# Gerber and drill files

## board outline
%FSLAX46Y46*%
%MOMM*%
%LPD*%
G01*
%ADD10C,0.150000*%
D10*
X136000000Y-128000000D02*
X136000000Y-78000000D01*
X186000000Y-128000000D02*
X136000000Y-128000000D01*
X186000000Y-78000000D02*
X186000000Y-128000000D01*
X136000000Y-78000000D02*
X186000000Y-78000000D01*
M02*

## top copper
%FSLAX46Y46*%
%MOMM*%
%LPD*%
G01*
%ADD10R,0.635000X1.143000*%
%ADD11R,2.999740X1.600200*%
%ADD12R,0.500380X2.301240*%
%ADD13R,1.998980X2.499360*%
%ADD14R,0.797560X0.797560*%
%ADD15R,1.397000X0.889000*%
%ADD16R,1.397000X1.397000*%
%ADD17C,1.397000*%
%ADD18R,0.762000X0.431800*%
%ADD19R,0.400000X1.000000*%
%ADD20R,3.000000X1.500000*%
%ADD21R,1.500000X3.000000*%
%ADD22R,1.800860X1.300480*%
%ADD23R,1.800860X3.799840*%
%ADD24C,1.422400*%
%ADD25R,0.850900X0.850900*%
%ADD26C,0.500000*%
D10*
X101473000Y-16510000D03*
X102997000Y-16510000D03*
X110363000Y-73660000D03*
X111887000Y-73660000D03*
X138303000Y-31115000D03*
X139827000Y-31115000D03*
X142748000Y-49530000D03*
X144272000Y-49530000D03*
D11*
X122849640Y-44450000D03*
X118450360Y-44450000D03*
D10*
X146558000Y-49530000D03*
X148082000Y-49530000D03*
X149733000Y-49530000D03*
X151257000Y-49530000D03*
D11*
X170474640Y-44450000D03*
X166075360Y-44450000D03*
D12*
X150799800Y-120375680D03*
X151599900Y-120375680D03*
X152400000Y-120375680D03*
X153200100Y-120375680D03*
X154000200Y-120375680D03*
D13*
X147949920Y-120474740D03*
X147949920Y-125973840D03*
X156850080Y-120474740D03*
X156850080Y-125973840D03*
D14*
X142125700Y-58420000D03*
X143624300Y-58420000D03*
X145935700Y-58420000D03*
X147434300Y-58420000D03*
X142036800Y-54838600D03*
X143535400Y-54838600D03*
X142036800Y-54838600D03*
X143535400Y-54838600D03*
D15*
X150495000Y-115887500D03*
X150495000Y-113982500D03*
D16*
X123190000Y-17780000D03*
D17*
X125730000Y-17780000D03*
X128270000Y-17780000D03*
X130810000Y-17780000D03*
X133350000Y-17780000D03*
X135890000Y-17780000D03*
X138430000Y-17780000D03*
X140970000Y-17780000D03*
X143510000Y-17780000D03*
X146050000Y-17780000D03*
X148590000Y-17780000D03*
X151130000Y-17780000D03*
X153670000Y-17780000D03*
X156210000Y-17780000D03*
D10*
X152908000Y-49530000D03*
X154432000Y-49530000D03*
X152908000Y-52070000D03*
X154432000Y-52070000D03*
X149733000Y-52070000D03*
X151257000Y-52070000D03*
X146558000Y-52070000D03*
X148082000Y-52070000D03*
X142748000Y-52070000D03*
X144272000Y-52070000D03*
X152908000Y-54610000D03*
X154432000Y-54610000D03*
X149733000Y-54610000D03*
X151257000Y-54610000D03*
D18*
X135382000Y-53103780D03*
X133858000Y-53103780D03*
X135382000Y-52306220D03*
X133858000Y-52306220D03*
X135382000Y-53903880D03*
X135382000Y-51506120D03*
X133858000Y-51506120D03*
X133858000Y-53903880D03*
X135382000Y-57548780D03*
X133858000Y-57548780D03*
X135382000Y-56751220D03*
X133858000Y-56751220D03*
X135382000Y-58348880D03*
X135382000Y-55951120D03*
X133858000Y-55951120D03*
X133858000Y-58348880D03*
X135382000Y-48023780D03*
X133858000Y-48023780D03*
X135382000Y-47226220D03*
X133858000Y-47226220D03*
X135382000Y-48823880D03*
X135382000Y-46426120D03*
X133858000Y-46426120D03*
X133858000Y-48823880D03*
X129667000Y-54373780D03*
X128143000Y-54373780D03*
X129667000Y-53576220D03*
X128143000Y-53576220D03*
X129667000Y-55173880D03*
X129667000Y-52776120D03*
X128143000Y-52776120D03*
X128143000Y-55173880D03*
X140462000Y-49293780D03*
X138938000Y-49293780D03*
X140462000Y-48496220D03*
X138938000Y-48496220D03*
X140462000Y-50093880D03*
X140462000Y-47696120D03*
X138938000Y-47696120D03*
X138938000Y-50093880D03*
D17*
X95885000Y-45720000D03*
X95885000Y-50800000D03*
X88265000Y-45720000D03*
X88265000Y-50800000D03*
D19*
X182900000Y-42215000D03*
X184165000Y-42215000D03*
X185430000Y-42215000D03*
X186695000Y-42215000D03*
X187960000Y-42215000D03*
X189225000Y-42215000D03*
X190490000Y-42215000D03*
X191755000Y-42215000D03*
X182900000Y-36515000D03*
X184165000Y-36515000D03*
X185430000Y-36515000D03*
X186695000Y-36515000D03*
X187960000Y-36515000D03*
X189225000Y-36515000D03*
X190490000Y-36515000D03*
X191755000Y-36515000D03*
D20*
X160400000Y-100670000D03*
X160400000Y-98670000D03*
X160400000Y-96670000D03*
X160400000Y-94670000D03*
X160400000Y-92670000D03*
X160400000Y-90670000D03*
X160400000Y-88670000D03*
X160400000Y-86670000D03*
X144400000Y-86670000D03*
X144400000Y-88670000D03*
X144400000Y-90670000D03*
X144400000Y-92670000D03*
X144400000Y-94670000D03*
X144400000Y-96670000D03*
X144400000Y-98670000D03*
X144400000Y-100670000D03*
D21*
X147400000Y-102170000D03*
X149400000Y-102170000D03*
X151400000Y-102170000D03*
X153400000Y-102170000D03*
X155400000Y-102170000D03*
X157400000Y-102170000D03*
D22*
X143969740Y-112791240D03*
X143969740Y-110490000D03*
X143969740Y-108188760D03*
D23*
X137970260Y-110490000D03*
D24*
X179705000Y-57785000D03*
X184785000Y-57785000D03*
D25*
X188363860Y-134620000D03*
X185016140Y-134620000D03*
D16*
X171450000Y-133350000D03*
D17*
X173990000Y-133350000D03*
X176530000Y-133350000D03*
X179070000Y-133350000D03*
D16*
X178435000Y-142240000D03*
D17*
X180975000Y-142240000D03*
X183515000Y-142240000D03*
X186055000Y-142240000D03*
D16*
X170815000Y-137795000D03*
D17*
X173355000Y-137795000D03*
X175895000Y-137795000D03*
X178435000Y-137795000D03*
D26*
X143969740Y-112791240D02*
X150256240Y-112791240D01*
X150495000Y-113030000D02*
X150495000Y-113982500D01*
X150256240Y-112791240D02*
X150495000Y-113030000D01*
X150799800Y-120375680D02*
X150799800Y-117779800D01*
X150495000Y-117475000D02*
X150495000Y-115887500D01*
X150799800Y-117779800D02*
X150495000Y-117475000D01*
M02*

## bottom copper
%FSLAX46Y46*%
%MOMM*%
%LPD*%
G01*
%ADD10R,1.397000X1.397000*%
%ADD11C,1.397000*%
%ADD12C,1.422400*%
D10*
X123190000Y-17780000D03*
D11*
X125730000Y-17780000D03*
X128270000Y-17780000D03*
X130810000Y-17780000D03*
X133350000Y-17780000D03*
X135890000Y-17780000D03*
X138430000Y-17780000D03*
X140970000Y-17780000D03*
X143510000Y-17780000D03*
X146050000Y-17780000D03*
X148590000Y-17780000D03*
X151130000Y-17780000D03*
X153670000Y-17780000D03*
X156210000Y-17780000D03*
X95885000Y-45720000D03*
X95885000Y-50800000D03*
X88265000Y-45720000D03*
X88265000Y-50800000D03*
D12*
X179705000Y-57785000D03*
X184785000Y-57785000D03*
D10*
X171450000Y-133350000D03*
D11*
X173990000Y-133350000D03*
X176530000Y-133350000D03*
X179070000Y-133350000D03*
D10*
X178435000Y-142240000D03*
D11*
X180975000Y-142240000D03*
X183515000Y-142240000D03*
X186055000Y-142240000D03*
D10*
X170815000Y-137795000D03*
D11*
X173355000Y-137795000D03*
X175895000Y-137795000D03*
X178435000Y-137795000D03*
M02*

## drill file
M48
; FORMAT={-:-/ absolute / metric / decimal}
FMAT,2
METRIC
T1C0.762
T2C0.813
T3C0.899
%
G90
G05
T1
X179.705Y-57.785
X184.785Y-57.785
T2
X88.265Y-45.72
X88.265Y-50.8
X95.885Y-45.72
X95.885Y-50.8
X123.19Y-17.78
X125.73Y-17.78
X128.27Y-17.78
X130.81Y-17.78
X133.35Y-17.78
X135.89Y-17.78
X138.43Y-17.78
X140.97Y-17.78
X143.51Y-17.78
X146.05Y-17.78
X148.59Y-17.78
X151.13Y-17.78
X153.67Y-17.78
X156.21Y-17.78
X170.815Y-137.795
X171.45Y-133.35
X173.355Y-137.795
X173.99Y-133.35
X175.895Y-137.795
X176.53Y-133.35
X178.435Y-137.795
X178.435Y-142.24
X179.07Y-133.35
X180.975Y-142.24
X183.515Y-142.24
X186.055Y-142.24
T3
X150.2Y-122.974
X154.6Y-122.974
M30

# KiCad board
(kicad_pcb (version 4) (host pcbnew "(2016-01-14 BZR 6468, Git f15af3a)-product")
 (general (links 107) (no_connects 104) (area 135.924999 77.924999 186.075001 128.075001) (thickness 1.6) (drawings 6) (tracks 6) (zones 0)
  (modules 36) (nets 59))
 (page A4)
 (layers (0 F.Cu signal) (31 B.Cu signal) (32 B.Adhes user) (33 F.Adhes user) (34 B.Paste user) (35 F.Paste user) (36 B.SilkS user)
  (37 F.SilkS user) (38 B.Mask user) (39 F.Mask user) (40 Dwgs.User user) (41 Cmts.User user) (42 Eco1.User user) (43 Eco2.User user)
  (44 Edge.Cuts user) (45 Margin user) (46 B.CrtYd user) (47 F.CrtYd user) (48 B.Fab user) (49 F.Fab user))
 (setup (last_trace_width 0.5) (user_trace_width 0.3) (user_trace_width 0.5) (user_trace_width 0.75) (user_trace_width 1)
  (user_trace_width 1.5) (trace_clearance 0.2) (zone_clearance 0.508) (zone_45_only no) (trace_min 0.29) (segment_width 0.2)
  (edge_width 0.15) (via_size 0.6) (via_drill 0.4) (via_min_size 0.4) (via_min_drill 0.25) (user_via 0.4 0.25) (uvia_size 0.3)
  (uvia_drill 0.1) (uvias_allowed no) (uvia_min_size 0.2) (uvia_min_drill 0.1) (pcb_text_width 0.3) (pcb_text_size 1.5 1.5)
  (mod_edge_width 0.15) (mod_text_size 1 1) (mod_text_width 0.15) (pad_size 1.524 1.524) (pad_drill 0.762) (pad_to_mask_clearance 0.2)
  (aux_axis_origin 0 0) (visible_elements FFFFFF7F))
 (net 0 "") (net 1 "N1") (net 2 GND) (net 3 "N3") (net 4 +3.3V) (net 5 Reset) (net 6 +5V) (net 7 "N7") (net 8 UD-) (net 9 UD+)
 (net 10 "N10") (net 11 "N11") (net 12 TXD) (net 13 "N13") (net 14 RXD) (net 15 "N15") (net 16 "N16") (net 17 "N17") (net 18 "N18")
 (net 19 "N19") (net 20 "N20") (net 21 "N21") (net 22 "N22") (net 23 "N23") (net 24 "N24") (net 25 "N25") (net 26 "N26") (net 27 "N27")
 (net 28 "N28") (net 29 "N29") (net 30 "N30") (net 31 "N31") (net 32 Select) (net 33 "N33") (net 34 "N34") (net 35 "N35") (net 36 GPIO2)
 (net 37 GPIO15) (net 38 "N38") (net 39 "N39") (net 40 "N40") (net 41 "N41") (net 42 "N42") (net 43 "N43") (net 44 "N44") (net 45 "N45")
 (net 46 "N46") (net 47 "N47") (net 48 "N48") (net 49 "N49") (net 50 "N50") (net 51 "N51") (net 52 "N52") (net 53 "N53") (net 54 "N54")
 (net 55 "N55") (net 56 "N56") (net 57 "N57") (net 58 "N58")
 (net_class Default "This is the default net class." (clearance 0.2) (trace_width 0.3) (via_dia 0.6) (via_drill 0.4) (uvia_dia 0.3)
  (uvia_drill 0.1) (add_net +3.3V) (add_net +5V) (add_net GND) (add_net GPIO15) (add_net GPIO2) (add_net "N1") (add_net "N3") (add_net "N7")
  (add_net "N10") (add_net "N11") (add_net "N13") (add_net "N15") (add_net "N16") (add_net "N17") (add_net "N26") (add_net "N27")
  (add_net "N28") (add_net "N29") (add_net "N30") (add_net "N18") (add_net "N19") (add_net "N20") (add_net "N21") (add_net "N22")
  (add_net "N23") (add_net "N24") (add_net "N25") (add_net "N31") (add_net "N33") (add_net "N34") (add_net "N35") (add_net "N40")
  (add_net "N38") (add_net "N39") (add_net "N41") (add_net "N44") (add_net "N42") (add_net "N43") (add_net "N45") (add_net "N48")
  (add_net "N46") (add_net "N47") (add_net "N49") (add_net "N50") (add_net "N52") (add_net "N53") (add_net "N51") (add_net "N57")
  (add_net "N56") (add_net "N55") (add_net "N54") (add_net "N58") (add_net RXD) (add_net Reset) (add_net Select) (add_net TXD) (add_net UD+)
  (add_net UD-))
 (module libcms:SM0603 (layer F.Cu) (at 102.235 16.51)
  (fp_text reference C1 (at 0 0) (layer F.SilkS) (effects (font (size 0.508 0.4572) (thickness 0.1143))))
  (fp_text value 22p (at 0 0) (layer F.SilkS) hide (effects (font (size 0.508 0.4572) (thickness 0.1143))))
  (pad 1 smd rect (at -0.762 0) (size 0.635 1.143) (layers F.Cu F.Paste F.Mask) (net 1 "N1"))
  (pad 2 smd rect (at 0.762 0) (size 0.635 1.143) (layers F.Cu F.Paste F.Mask) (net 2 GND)))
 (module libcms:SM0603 (layer F.Cu) (at 111.125 73.66)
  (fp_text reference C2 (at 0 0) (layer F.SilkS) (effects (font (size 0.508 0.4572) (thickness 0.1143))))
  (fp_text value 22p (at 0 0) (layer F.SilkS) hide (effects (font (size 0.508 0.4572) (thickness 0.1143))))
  (pad 1 smd rect (at -0.762 0) (size 0.635 1.143) (layers F.Cu F.Paste F.Mask) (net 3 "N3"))
  (pad 2 smd rect (at 0.762 0) (size 0.635 1.143) (layers F.Cu F.Paste F.Mask) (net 2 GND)))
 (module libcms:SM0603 (layer F.Cu) (at 139.065 31.115)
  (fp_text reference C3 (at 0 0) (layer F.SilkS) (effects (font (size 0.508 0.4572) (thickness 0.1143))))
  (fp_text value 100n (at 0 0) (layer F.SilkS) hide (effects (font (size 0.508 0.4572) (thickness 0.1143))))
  (pad 1 smd rect (at -0.762 0) (size 0.635 1.143) (layers F.Cu F.Paste F.Mask) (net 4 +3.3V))
  (pad 2 smd rect (at 0.762 0) (size 0.635 1.143) (layers F.Cu F.Paste F.Mask) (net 2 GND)))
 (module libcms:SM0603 (layer F.Cu) (at 143.51 49.53)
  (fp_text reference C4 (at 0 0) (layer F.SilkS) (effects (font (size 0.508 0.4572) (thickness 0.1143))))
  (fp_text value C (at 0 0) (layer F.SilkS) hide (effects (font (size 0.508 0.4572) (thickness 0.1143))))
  (pad 1 smd rect (at -0.762 0) (size 0.635 1.143) (layers F.Cu F.Paste F.Mask) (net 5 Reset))
  (pad 2 smd rect (at 0.762 0) (size 0.635 1.143) (layers F.Cu F.Paste F.Mask) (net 2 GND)))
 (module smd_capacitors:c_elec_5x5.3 (layer F.Cu) (at 120.65 44.45)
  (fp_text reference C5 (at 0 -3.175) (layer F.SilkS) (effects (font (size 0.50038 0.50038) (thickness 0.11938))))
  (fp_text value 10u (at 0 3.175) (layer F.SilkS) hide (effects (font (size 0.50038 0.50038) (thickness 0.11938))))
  (pad 1 smd rect (at 2.19964 0) (size 2.99974 1.6002) (layers F.Cu F.Paste F.Mask) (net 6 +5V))
  (pad 2 smd rect (at -2.19964 0) (size 2.99974 1.6002) (layers F.Cu F.Paste F.Mask) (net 2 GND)))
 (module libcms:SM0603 (layer F.Cu) (at 147.32 49.53)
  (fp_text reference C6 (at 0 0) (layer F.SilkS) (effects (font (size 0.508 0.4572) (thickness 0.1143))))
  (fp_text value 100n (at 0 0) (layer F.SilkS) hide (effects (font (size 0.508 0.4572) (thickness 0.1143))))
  (pad 1 smd rect (at -0.762 0) (size 0.635 1.143) (layers F.Cu F.Paste F.Mask) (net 6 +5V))
  (pad 2 smd rect (at 0.762 0) (size 0.635 1.143) (layers F.Cu F.Paste F.Mask) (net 2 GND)))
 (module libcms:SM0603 (layer F.Cu) (at 150.495 49.53)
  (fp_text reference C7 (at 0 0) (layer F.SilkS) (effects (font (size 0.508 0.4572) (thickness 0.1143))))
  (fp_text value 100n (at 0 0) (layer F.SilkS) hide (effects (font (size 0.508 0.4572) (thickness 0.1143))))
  (pad 1 smd rect (at -0.762 0) (size 0.635 1.143) (layers F.Cu F.Paste F.Mask) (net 4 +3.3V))
  (pad 2 smd rect (at 0.762 0) (size 0.635 1.143) (layers F.Cu F.Paste F.Mask) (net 2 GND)))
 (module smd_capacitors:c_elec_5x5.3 (layer F.Cu) (at 168.275 44.45)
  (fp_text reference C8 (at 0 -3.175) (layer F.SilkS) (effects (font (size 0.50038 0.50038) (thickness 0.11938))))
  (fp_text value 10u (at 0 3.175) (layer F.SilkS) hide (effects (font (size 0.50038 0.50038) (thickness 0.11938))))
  (pad 1 smd rect (at 2.19964 0) (size 2.99974 1.6002) (layers F.Cu F.Paste F.Mask) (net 4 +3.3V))
  (pad 2 smd rect (at -2.19964 0) (size 2.99974 1.6002) (layers F.Cu F.Paste F.Mask) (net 2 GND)))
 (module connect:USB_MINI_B (layer F.Cu) (at 152.4 123.825 90)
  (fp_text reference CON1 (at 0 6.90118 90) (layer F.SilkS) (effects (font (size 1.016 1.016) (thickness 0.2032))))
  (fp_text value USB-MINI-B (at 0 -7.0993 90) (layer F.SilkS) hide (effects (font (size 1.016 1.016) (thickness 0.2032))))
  (pad 1 smd rect (at 3.44932 -1.6002 90) (size 2.30124 0.50038) (layers F.Cu F.Paste F.Mask) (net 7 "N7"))
  (pad 2 smd rect (at 3.44932 -0.8001 90) (size 2.30124 0.50038) (layers F.Cu F.Paste F.Mask) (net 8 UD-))
  (pad 3 smd rect (at 3.44932 0 90) (size 2.30124 0.50038) (layers F.Cu F.Paste F.Mask) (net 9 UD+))
  (pad 4 smd rect (at 3.44932 0.8001 90) (size 2.30124 0.50038) (layers F.Cu F.Paste F.Mask) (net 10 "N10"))
  (pad 5 smd rect (at 3.44932 1.6002 90) (size 2.30124 0.50038) (layers F.Cu F.Paste F.Mask) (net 2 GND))
  (pad 6 smd rect (at 3.35026 -4.45008 90) (size 2.49936 1.99898) (layers F.Cu F.Paste F.Mask) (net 2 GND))
  (pad 7 smd rect (at -2.14884 -4.45008 90) (size 2.49936 1.99898) (layers F.Cu F.Paste F.Mask) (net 2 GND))
  (pad 8 smd rect (at 3.35026 4.45008 90) (size 2.49936 1.99898) (layers F.Cu F.Paste F.Mask) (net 2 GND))
  (pad 9 smd rect (at -2.14884 4.45008 90) (size 2.49936 1.99898) (layers F.Cu F.Paste F.Mask) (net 2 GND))
  (pad "" np_thru_hole circle (at 0.8509 -2.19964 90) (size 0.89916 0.89916) (drill 0.89916) (layers *.Cu *.Mask F.SilkS))
  (pad 2 np_thru_hole circle (at 0.8509 2.19964 90) (size 0.89916 0.89916) (drill 0.89916) (layers *.Cu *.Mask F.SilkS) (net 8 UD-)))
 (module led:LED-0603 (layer F.Cu) (at 142.875 58.42)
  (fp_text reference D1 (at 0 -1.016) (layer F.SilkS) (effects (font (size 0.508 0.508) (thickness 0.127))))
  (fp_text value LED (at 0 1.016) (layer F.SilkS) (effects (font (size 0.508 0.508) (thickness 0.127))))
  (pad 1 smd rect (at -0.7493 0) (size 0.79756 0.79756) (layers F.Cu F.Paste F.Mask) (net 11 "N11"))
  (pad 2 smd rect (at 0.7493 0) (size 0.79756 0.79756) (layers F.Cu F.Paste F.Mask) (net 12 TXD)))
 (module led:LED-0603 (layer F.Cu) (at 146.685 58.42)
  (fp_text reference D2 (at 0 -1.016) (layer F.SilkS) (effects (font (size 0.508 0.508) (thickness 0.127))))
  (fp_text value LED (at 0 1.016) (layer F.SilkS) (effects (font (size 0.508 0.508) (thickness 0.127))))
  (pad 1 smd rect (at -0.7493 0) (size 0.79756 0.79756) (layers F.Cu F.Paste F.Mask) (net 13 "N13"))
  (pad 2 smd rect (at 0.7493 0) (size 0.79756 0.79756) (layers F.Cu F.Paste F.Mask) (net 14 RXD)))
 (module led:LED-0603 (layer F.Cu) (at 142.7861 54.8386)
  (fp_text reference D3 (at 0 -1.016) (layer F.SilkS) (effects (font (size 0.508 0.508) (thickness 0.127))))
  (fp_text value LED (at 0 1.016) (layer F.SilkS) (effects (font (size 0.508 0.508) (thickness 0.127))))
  (pad 1 smd rect (at -0.7493 0) (size 0.79756 0.79756) (layers F.Cu F.Paste F.Mask) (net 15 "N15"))
  (pad 2 smd rect (at 0.7493 0) (size 0.79756 0.79756) (layers F.Cu F.Paste F.Mask) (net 2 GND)))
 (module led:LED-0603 (layer F.Cu) (at 142.7861 54.8386)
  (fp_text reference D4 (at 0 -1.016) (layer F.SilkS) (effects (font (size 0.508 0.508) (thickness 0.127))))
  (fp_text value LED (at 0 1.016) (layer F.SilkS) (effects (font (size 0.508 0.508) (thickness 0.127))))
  (pad 1 smd rect (at -0.7493 0) (size 0.79756 0.79756) (layers F.Cu F.Paste F.Mask) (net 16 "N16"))
  (pad 2 smd rect (at 0.7493 0) (size 0.79756 0.79756) (layers F.Cu F.Paste F.Mask) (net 2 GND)))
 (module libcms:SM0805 (layer F.Cu) (at 150.495 114.935 90)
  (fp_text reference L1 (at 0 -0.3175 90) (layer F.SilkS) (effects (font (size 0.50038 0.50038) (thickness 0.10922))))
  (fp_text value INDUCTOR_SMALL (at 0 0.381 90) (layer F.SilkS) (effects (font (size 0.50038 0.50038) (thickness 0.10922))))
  (pad 1 smd rect (at -0.9525 0 90) (size 0.889 1.397) (layers F.Cu F.Paste F.Mask) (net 7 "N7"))
  (pad 2 smd rect (at 0.9525 0 90) (size 0.889 1.397) (layers F.Cu F.Paste F.Mask) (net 6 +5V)))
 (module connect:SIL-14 (layer F.Cu) (at 139.7 17.78)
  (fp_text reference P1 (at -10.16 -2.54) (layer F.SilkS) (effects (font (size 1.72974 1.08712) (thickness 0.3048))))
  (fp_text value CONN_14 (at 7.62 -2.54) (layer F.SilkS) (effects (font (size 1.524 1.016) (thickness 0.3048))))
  (pad 1 thru_hole rect (at -16.51 0) (size 1.397 1.397) (drill 0.8128) (layers *.Cu *.Mask F.SilkS) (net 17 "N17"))
  (pad 2 thru_hole circle (at -13.97 0) (size 1.397 1.397) (drill 0.8128) (layers *.Cu *.Mask F.SilkS) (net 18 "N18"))
  (pad 3 thru_hole circle (at -11.43 0) (size 1.397 1.397) (drill 0.8128) (layers *.Cu *.Mask F.SilkS) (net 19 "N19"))
  (pad 4 thru_hole circle (at -8.89 0) (size 1.397 1.397) (drill 0.8128) (layers *.Cu *.Mask F.SilkS) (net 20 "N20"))
  (pad 5 thru_hole circle (at -6.35 0) (size 1.397 1.397) (drill 0.8128) (layers *.Cu *.Mask F.SilkS) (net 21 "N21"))
  (pad 6 thru_hole circle (at -3.81 0) (size 1.397 1.397) (drill 0.8128) (layers *.Cu *.Mask F.SilkS) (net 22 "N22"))
  (pad 7 thru_hole circle (at -1.27 0) (size 1.397 1.397) (drill 0.8128) (layers *.Cu *.Mask F.SilkS) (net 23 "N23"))
  (pad 8 thru_hole circle (at 1.27 0) (size 1.397 1.397) (drill 0.8128) (layers *.Cu *.Mask F.SilkS) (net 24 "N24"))
  (pad 9 thru_hole circle (at 3.81 0) (size 1.397 1.397) (drill 0.8128) (layers *.Cu *.Mask F.SilkS) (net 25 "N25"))
  (pad 10 thru_hole circle (at 6.35 0) (size 1.397 1.397) (drill 0.8128) (layers *.Cu *.Mask F.SilkS) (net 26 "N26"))
  (pad 11 thru_hole circle (at 8.89 0) (size 1.397 1.397) (drill 0.8128) (layers *.Cu *.Mask F.SilkS) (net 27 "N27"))
  (pad 12 thru_hole circle (at 11.43 0) (size 1.397 1.397) (drill 0.8128) (layers *.Cu *.Mask F.SilkS) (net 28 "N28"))
  (pad 13 thru_hole circle (at 13.97 0) (size 1.397 1.397) (drill 0.8128) (layers *.Cu *.Mask F.SilkS) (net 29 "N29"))
  (pad 14 thru_hole circle (at 16.51 0) (size 1.397 1.397) (drill 0.8128) (layers *.Cu *.Mask F.SilkS) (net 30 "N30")))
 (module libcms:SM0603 (layer F.Cu) (at 153.67 49.53)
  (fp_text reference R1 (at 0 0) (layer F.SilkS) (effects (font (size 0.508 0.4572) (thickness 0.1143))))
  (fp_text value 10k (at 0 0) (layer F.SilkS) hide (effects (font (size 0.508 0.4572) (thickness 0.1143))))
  (pad 1 smd rect (at -0.762 0) (size 0.635 1.143) (layers F.Cu F.Paste F.Mask) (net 5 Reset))
  (pad 2 smd rect (at 0.762 0) (size 0.635 1.143) (layers F.Cu F.Paste F.Mask) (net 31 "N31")))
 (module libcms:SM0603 (layer F.Cu) (at 153.67 52.07)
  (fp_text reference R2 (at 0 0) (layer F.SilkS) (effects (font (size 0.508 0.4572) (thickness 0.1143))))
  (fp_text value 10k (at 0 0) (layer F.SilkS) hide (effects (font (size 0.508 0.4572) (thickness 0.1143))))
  (pad 1 smd rect (at -0.762 0) (size 0.635 1.143) (layers F.Cu F.Paste F.Mask) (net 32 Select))
  (pad 2 smd rect (at 0.762 0) (size 0.635 1.143) (layers F.Cu F.Paste F.Mask) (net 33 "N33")))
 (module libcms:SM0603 (layer F.Cu) (at 150.495 52.07)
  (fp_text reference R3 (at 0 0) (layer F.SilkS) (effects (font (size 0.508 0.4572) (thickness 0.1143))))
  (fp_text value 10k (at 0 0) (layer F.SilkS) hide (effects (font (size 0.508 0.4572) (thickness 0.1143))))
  (pad 1 smd rect (at -0.762 0) (size 0.635 1.143) (layers F.Cu F.Paste F.Mask) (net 5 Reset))
  (pad 2 smd rect (at 0.762 0) (size 0.635 1.143) (layers F.Cu F.Paste F.Mask) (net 4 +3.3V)))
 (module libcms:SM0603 (layer F.Cu) (at 147.32 52.07)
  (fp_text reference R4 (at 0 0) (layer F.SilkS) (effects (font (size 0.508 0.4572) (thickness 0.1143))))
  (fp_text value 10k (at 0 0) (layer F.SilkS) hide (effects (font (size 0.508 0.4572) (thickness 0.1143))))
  (pad 1 smd rect (at -0.762 0) (size 0.635 1.143) (layers F.Cu F.Paste F.Mask) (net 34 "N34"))
  (pad 2 smd rect (at 0.762 0) (size 0.635 1.143) (layers F.Cu F.Paste F.Mask) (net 5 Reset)))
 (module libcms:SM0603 (layer F.Cu) (at 143.51 52.07)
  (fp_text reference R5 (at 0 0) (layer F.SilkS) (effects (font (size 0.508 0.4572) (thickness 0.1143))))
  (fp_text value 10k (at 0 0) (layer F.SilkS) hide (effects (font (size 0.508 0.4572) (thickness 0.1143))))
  (pad 1 smd rect (at -0.762 0) (size 0.635 1.143) (layers F.Cu F.Paste F.Mask) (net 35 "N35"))
  (pad 2 smd rect (at 0.762 0) (size 0.635 1.143) (layers F.Cu F.Paste F.Mask) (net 4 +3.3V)))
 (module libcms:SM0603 (layer F.Cu) (at 153.67 54.61)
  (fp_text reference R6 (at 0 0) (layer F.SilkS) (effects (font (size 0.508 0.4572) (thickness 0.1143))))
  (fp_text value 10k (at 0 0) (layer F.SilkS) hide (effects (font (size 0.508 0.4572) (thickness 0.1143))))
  (pad 1 smd rect (at -0.762 0) (size 0.635 1.143) (layers F.Cu F.Paste F.Mask) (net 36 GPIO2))
  (pad 2 smd rect (at 0.762 0) (size 0.635 1.143) (layers F.Cu F.Paste F.Mask) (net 4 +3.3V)))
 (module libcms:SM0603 (layer F.Cu) (at 150.495 54.61)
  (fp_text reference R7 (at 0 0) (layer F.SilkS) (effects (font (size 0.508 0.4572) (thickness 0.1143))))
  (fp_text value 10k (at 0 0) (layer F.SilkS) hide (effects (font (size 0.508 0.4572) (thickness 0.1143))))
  (pad 1 smd rect (at -0.762 0) (size 0.635 1.143) (layers F.Cu F.Paste F.Mask) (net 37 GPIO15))
  (pad 2 smd rect (at 0.762 0) (size 0.635 1.143) (layers F.Cu F.Paste F.Mask) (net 2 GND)))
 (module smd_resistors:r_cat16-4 (layer F.Cu) (at 134.62 52.705)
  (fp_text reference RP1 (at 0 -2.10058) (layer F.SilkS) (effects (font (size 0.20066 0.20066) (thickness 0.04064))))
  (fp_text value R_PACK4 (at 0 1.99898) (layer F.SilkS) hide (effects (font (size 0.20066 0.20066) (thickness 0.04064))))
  (pad 2 smd rect (at 0.762 0.39878) (size 0.762 0.4318) (layers F.Cu F.Paste F.Mask) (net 4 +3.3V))
  (pad 7 smd rect (at -0.762 0.39878) (size 0.762 0.4318) (layers F.Cu F.Paste F.Mask) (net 15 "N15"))
  (pad 3 smd rect (at 0.762 -0.39878) (size 0.762 0.4318) (layers F.Cu F.Paste F.Mask) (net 4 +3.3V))
  (pad 6 smd rect (at -0.762 -0.39878) (size 0.762 0.4318) (layers F.Cu F.Paste F.Mask) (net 13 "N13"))
  (pad 1 smd rect (at 0.762 1.19888) (size 0.762 0.4318) (layers F.Cu F.Paste F.Mask) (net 6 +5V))
  (pad 4 smd rect (at 0.762 -1.19888) (size 0.762 0.4318) (layers F.Cu F.Paste F.Mask) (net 4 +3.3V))
  (pad 5 smd rect (at -0.762 -1.19888) (size 0.762 0.4318) (layers F.Cu F.Paste F.Mask) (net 11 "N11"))
  (pad 8 smd rect (at -0.762 1.19888) (size 0.762 0.4318) (layers F.Cu F.Paste F.Mask) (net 16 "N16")))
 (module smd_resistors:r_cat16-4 (layer F.Cu) (at 134.62 57.15)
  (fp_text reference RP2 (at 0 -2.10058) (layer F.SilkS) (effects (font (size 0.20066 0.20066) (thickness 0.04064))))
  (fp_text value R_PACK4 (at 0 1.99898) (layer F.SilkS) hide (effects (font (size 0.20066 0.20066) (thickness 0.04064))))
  (pad 2 smd rect (at 0.762 0.39878) (size 0.762 0.4318) (layers F.Cu F.Paste F.Mask) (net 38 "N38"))
  (pad 7 smd rect (at -0.762 0.39878) (size 0.762 0.4318) (layers F.Cu F.Paste F.Mask) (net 18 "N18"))
  (pad 3 smd rect (at 0.762 -0.39878) (size 0.762 0.4318) (layers F.Cu F.Paste F.Mask) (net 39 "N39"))
  (pad 6 smd rect (at -0.762 -0.39878) (size 0.762 0.4318) (layers F.Cu F.Paste F.Mask) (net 19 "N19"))
  (pad 1 smd rect (at 0.762 1.19888) (size 0.762 0.4318) (layers F.Cu F.Paste F.Mask) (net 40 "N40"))
  (pad 4 smd rect (at 0.762 -1.19888) (size 0.762 0.4318) (layers F.Cu F.Paste F.Mask) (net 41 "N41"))
  (pad 5 smd rect (at -0.762 -1.19888) (size 0.762 0.4318) (layers F.Cu F.Paste F.Mask) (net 20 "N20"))
  (pad 8 smd rect (at -0.762 1.19888) (size 0.762 0.4318) (layers F.Cu F.Paste F.Mask) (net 17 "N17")))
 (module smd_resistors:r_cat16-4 (layer F.Cu) (at 134.62 47.625)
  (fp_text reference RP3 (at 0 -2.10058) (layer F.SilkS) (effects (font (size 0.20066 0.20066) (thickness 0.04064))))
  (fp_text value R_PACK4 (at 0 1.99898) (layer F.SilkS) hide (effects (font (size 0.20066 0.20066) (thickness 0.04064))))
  (pad 2 smd rect (at 0.762 0.39878) (size 0.762 0.4318) (layers F.Cu F.Paste F.Mask) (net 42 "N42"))
  (pad 7 smd rect (at -0.762 0.39878) (size 0.762 0.4318) (layers F.Cu F.Paste F.Mask) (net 22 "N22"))
  (pad 3 smd rect (at 0.762 -0.39878) (size 0.762 0.4318) (layers F.Cu F.Paste F.Mask) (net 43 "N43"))
  (pad 6 smd rect (at -0.762 -0.39878) (size 0.762 0.4318) (layers F.Cu F.Paste F.Mask) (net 23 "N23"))
  (pad 1 smd rect (at 0.762 1.19888) (size 0.762 0.4318) (layers F.Cu F.Paste F.Mask) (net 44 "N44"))
  (pad 4 smd rect (at 0.762 -1.19888) (size 0.762 0.4318) (layers F.Cu F.Paste F.Mask) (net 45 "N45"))
  (pad 5 smd rect (at -0.762 -1.19888) (size 0.762 0.4318) (layers F.Cu F.Paste F.Mask) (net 24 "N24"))
  (pad 8 smd rect (at -0.762 1.19888) (size 0.762 0.4318) (layers F.Cu F.Paste F.Mask) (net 21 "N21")))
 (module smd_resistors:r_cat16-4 (layer F.Cu) (at 128.905 53.975)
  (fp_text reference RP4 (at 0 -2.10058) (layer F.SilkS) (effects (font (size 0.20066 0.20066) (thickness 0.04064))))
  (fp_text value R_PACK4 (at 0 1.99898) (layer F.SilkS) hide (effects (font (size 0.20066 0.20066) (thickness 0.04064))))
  (pad 2 smd rect (at 0.762 0.39878) (size 0.762 0.4318) (layers F.Cu F.Paste F.Mask) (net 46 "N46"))
  (pad 7 smd rect (at -0.762 0.39878) (size 0.762 0.4318) (layers F.Cu F.Paste F.Mask) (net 26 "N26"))
  (pad 3 smd rect (at 0.762 -0.39878) (size 0.762 0.4318) (layers F.Cu F.Paste F.Mask) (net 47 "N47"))
  (pad 6 smd rect (at -0.762 -0.39878) (size 0.762 0.4318) (layers F.Cu F.Paste F.Mask) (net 27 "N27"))
  (pad 1 smd rect (at 0.762 1.19888) (size 0.762 0.4318) (layers F.Cu F.Paste F.Mask) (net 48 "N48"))
  (pad 4 smd rect (at 0.762 -1.19888) (size 0.762 0.4318) (layers F.Cu F.Paste F.Mask) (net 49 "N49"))
  (pad 5 smd rect (at -0.762 -1.19888) (size 0.762 0.4318) (layers F.Cu F.Paste F.Mask) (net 28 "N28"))
  (pad 8 smd rect (at -0.762 1.19888) (size 0.762 0.4318) (layers F.Cu F.Paste F.Mask) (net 25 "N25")))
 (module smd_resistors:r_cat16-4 (layer F.Cu) (at 139.7 48.895)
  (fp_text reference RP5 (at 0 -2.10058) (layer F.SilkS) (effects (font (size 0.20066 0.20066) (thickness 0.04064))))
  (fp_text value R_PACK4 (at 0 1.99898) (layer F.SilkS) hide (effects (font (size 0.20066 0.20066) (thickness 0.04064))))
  (pad 2 smd rect (at 0.762 0.39878) (size 0.762 0.4318) (layers F.Cu F.Paste F.Mask) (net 37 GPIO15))
  (pad 7 smd rect (at -0.762 0.39878) (size 0.762 0.4318) (layers F.Cu F.Paste F.Mask) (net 30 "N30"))
  (pad 3 smd rect (at 0.762 -0.39878) (size 0.762 0.4318) (layers F.Cu F.Paste F.Mask) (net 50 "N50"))
  (pad 6 smd rect (at -0.762 -0.39878) (size 0.762 0.4318) (layers F.Cu F.Paste F.Mask) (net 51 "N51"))
  (pad 1 smd rect (at 0.762 1.19888) (size 0.762 0.4318) (layers F.Cu F.Paste F.Mask) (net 36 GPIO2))
  (pad 4 smd rect (at 0.762 -1.19888) (size 0.762 0.4318) (layers F.Cu F.Paste F.Mask) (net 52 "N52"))
  (pad 5 smd rect (at -0.762 -1.19888) (size 0.762 0.4318) (layers F.Cu F.Paste F.Mask) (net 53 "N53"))
  (pad 8 smd rect (at -0.762 1.19888) (size 0.762 0.4318) (layers F.Cu F.Paste F.Mask) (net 29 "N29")))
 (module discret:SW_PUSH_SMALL (layer F.Cu) (at 92.075 48.26)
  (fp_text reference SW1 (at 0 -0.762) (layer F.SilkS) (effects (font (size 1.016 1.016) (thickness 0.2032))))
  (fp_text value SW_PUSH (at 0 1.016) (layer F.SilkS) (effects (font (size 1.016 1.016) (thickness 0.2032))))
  (pad 1 thru_hole circle (at 3.81 -2.54) (size 1.397 1.397) (drill 0.8128) (layers *.Cu *.Mask F.SilkS) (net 2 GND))
  (pad 2 thru_hole circle (at 3.81 2.54) (size 1.397 1.397) (drill 0.8128) (layers *.Cu *.Mask F.SilkS) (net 5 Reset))
  (pad 1 thru_hole circle (at -3.81 -2.54) (size 1.397 1.397) (drill 0.8128) (layers *.Cu *.Mask F.SilkS) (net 2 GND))
  (pad 2 thru_hole circle (at -3.81 2.54) (size 1.397 1.397) (drill 0.8128) (layers *.Cu *.Mask F.SilkS) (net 5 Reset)))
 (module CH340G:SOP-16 (layer F.Cu) (at 187.325 39.37) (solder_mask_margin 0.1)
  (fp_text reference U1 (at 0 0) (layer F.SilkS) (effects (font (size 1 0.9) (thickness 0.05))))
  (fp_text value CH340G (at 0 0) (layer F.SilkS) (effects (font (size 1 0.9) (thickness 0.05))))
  (pad 1 smd rect (at -4.425 2.845 180) (size 0.4 1) (layers F.Cu F.Paste F.Mask) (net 2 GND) (solder_mask_margin 0.2))
  (pad 2 smd rect (at -3.16 2.845 180) (size 0.4 1) (layers F.Cu F.Paste F.Mask) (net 12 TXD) (solder_mask_margin 0.2))
  (pad 3 smd rect (at -1.895 2.845 180) (size 0.4 1) (layers F.Cu F.Paste F.Mask) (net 14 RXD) (solder_mask_margin 0.2))
  (pad 4 smd rect (at -0.63 2.845 180) (size 0.4 1) (layers F.Cu F.Paste F.Mask) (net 4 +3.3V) (solder_mask_margin 0.2))
  (pad 5 smd rect (at 0.635 2.845 180) (size 0.4 1) (layers F.Cu F.Paste F.Mask) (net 9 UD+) (solder_mask_margin 0.2))
  (pad 6 smd rect (at 1.9 2.845 180) (size 0.4 1) (layers F.Cu F.Paste F.Mask) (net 8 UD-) (solder_mask_margin 0.2))
  (pad 7 smd rect (at 3.165 2.845 180) (size 0.4 1) (layers F.Cu F.Paste F.Mask) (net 1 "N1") (solder_mask_margin 0.2))
  (pad 8 smd rect (at 4.43 2.845 180) (size 0.4 1) (layers F.Cu F.Paste F.Mask) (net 3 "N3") (solder_mask_margin 0.2))
  (pad 16 smd rect (at -4.425 -2.855 180) (size 0.4 1) (layers F.Cu F.Paste F.Mask) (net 4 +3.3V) (solder_mask_margin 0.2))
  (pad 15 smd rect (at -3.16 -2.855 180) (size 0.4 1) (layers F.Cu F.Paste F.Mask) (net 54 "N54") (solder_mask_margin 0.2))
  (pad 14 smd rect (at -1.895 -2.855 180) (size 0.4 1) (layers F.Cu F.Paste F.Mask) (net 31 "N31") (solder_mask_margin 0.2))
  (pad 13 smd rect (at -0.63 -2.855 180) (size 0.4 1) (layers F.Cu F.Paste F.Mask) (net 33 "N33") (solder_mask_margin 0.2))
  (pad 12 smd rect (at 0.635 -2.855 180) (size 0.4 1) (layers F.Cu F.Paste F.Mask) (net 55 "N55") (solder_mask_margin 0.2))
  (pad 11 smd rect (at 1.9 -2.855 180) (size 0.4 1) (layers F.Cu F.Paste F.Mask) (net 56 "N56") (solder_mask_margin 0.2))
  (pad 10 smd rect (at 3.165 -2.855 180) (size 0.4 1) (layers F.Cu F.Paste F.Mask) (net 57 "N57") (solder_mask_margin 0.2))
  (pad 9 smd rect (at 4.43 -2.855 180) (size 0.4 1) (layers F.Cu F.Paste F.Mask) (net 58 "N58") (solder_mask_margin 0.2)))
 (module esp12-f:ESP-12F (layer F.Cu) (at 152.4 90.17)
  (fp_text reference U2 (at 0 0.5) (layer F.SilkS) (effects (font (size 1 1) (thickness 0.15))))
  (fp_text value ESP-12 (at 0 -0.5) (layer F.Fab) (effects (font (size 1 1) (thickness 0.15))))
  (pad 15 smd rect (at 8 10.5) (size 3 1.5) (layers F.Cu F.Paste F.Mask) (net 2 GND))
  (pad 16 smd rect (at 8 8.5) (size 3 1.5) (layers F.Cu F.Paste F.Mask) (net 37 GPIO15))
  (pad 17 smd rect (at 8 6.5) (size 3 1.5) (layers F.Cu F.Paste F.Mask) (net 36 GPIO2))
  (pad 18 smd rect (at 8 4.5) (size 3 1.5) (layers F.Cu F.Paste F.Mask) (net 32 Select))
  (pad 19 smd rect (at 8 2.5) (size 3 1.5) (layers F.Cu F.Paste F.Mask) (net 47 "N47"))
  (pad 20 smd rect (at 8 0.5) (size 3 1.5) (layers F.Cu F.Paste F.Mask) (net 49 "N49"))
  (pad 21 smd rect (at 8 -1.5) (size 3 1.5) (layers F.Cu F.Paste F.Mask) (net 12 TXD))
  (pad 22 smd rect (at 8 -3.5) (size 3 1.5) (layers F.Cu F.Paste F.Mask) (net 14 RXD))
  (pad 1 smd rect (at -8 -3.5) (size 3 1.5) (layers F.Cu F.Paste F.Mask) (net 5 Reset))
  (pad 2 smd rect (at -8 -1.5) (size 3 1.5) (layers F.Cu F.Paste F.Mask) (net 40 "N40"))
  (pad 3 smd rect (at -8 0.5) (size 3 1.5) (layers F.Cu F.Paste F.Mask) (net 35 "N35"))
  (pad 4 smd rect (at -8 2.5) (size 3 1.5) (layers F.Cu F.Paste F.Mask) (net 34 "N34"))
  (pad 5 smd rect (at -8 4.5) (size 3 1.5) (layers F.Cu F.Paste F.Mask) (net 38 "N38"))
  (pad 6 smd rect (at -8 6.5) (size 3 1.5) (layers F.Cu F.Paste F.Mask) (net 39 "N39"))
  (pad 7 smd rect (at -8 8.5) (size 3 1.5) (layers F.Cu F.Paste F.Mask) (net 41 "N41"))
  (pad 8 smd rect (at -8 10.5) (size 3 1.5) (layers F.Cu F.Paste F.Mask) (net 4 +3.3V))
  (pad 9 smd rect (at -5 12 90) (size 3 1.5) (layers F.Cu F.Paste F.Mask) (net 44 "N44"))
  (pad 10 smd rect (at -3 12 90) (size 3 1.5) (layers F.Cu F.Paste F.Mask) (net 42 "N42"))
  (pad 11 smd rect (at -1 12 90) (size 3 1.5) (layers F.Cu F.Paste F.Mask) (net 43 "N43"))
  (pad 12 smd rect (at 1 12 90) (size 3 1.5) (layers F.Cu F.Paste F.Mask) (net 45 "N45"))
  (pad 13 smd rect (at 3 12 90) (size 3 1.5) (layers F.Cu F.Paste F.Mask) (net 48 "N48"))
  (pad 14 smd rect (at 5 12 90) (size 3 1.5) (layers F.Cu F.Paste F.Mask) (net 46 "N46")))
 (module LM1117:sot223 (layer F.Cu) (at 140.97 110.49 90)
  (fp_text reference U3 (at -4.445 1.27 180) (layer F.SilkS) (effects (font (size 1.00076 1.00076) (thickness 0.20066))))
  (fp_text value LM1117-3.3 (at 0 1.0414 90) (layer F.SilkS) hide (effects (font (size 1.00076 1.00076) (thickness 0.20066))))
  (pad 1 smd rect (at -2.30124 2.99974 90) (size 1.30048 1.80086) (layers F.Cu F.Paste F.Mask) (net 6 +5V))
  (pad 2 smd rect (at 0 2.99974 90) (size 1.30048 1.80086) (layers F.Cu F.Paste F.Mask) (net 2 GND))
  (pad 3 smd rect (at 2.30124 2.99974 90) (size 1.30048 1.80086) (layers F.Cu F.Paste F.Mask) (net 4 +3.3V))
  (pad 4 smd rect (at 0 -2.99974 90) (size 3.79984 1.80086) (layers F.Cu F.Paste F.Mask)))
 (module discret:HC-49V (layer F.Cu) (at 182.245 57.785) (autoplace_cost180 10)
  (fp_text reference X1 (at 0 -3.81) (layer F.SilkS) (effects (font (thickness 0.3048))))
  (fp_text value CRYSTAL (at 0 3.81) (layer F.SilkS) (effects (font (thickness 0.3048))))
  (pad 1 thru_hole circle (at -2.54 0) (size 1.4224 1.4224) (drill 0.762) (layers *.Cu *.Mask F.SilkS) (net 1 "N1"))
  (pad 2 thru_hole circle (at 2.54 0) (size 1.4224 1.4224) (drill 0.762) (layers *.Cu *.Mask F.SilkS) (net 3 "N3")))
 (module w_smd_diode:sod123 (layer F.Cu) (at 186.69 134.62)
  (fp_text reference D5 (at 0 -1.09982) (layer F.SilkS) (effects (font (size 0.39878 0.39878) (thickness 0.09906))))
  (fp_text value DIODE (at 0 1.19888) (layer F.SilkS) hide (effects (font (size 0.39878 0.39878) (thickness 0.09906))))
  (pad 2 smd rect (at 1.67386 0) (size 0.8509 0.8509) (layers F.Cu F.Paste F.Mask) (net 6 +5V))
  (pad 1 smd rect (at -1.67386 0) (size 0.8509 0.8509) (layers F.Cu F.Paste F.Mask) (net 4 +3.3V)))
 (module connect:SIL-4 (layer F.Cu) (at 175.26 133.35)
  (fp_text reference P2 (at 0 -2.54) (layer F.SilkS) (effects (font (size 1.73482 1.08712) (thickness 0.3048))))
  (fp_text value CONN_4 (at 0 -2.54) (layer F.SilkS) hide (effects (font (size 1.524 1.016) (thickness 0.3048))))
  (pad 1 thru_hole rect (at -3.81 0) (size 1.397 1.397) (drill 0.8128) (layers *.Cu *.Mask F.SilkS) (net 6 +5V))
  (pad 2 thru_hole circle (at -1.27 0) (size 1.397 1.397) (drill 0.8128) (layers *.Cu *.Mask F.SilkS) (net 6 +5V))
  (pad 3 thru_hole circle (at 1.27 0) (size 1.397 1.397) (drill 0.8128) (layers *.Cu *.Mask F.SilkS) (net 6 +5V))
  (pad 4 thru_hole circle (at 3.81 0) (size 1.397 1.397) (drill 0.8128) (layers *.Cu *.Mask F.SilkS) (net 6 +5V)))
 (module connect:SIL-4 (layer F.Cu) (at 182.245 142.24)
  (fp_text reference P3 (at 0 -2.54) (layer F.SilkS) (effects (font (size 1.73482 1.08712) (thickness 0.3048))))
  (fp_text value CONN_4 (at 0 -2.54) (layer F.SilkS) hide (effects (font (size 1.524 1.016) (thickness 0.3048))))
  (pad 1 thru_hole rect (at -3.81 0) (size 1.397 1.397) (drill 0.8128) (layers *.Cu *.Mask F.SilkS) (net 4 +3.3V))
  (pad 2 thru_hole circle (at -1.27 0) (size 1.397 1.397) (drill 0.8128) (layers *.Cu *.Mask F.SilkS) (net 4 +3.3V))
  (pad 3 thru_hole circle (at 1.27 0) (size 1.397 1.397) (drill 0.8128) (layers *.Cu *.Mask F.SilkS) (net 4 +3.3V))
  (pad 4 thru_hole circle (at 3.81 0) (size 1.397 1.397) (drill 0.8128) (layers *.Cu *.Mask F.SilkS) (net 4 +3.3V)))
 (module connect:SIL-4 (layer F.Cu) (at 174.625 137.795)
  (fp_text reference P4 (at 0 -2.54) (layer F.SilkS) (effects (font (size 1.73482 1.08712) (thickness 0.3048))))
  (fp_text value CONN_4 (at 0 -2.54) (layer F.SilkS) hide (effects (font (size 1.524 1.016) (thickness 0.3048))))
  (pad 1 thru_hole rect (at -3.81 0) (size 1.397 1.397) (drill 0.8128) (layers *.Cu *.Mask F.SilkS) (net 2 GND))
  (pad 2 thru_hole circle (at -1.27 0) (size 1.397 1.397) (drill 0.8128) (layers *.Cu *.Mask F.SilkS) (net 2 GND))
  (pad 3 thru_hole circle (at 1.27 0) (size 1.397 1.397) (drill 0.8128) (layers *.Cu *.Mask F.SilkS) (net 2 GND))
  (pad 4 thru_hole circle (at 3.81 0) (size 1.397 1.397) (drill 0.8128) (layers *.Cu *.Mask F.SilkS) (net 2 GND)))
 (gr_line (start 136 128) (end 136 78) (angle 90) (layer Edge.Cuts) (width 0.15))
 (gr_line (start 186 128) (end 136 128) (angle 90) (layer Edge.Cuts) (width 0.15))
 (gr_line (start 186 78) (end 186 128) (angle 90) (layer Edge.Cuts) (width 0.15))
 (gr_line (start 136 78) (end 186 78) (angle 90) (layer Edge.Cuts) (width 0.15))
 (segment (start 143.96974 112.79124) (end 150.25624 112.79124) (width 0.5) (layer F.Cu) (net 6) (status 400000))
 (segment (start 150.495 113.03) (end 150.495 113.9825) (width 0.5) (layer F.Cu) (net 6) (status 800000))
 (segment (start 150.25624 112.79124) (end 150.495 113.03) (width 0.5) (layer F.Cu) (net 6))
 (segment (start 150.7998 120.37568) (end 150.7998 117.7798) (width 0.5) (layer F.Cu) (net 7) (status 400000))
 (segment (start 150.495 117.475) (end 150.495 115.8875) (width 0.5) (layer F.Cu) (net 7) (status 800000))
 (segment (start 150.7998 117.7798) (end 150.495 117.475) (width 0.5) (layer F.Cu) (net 7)))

